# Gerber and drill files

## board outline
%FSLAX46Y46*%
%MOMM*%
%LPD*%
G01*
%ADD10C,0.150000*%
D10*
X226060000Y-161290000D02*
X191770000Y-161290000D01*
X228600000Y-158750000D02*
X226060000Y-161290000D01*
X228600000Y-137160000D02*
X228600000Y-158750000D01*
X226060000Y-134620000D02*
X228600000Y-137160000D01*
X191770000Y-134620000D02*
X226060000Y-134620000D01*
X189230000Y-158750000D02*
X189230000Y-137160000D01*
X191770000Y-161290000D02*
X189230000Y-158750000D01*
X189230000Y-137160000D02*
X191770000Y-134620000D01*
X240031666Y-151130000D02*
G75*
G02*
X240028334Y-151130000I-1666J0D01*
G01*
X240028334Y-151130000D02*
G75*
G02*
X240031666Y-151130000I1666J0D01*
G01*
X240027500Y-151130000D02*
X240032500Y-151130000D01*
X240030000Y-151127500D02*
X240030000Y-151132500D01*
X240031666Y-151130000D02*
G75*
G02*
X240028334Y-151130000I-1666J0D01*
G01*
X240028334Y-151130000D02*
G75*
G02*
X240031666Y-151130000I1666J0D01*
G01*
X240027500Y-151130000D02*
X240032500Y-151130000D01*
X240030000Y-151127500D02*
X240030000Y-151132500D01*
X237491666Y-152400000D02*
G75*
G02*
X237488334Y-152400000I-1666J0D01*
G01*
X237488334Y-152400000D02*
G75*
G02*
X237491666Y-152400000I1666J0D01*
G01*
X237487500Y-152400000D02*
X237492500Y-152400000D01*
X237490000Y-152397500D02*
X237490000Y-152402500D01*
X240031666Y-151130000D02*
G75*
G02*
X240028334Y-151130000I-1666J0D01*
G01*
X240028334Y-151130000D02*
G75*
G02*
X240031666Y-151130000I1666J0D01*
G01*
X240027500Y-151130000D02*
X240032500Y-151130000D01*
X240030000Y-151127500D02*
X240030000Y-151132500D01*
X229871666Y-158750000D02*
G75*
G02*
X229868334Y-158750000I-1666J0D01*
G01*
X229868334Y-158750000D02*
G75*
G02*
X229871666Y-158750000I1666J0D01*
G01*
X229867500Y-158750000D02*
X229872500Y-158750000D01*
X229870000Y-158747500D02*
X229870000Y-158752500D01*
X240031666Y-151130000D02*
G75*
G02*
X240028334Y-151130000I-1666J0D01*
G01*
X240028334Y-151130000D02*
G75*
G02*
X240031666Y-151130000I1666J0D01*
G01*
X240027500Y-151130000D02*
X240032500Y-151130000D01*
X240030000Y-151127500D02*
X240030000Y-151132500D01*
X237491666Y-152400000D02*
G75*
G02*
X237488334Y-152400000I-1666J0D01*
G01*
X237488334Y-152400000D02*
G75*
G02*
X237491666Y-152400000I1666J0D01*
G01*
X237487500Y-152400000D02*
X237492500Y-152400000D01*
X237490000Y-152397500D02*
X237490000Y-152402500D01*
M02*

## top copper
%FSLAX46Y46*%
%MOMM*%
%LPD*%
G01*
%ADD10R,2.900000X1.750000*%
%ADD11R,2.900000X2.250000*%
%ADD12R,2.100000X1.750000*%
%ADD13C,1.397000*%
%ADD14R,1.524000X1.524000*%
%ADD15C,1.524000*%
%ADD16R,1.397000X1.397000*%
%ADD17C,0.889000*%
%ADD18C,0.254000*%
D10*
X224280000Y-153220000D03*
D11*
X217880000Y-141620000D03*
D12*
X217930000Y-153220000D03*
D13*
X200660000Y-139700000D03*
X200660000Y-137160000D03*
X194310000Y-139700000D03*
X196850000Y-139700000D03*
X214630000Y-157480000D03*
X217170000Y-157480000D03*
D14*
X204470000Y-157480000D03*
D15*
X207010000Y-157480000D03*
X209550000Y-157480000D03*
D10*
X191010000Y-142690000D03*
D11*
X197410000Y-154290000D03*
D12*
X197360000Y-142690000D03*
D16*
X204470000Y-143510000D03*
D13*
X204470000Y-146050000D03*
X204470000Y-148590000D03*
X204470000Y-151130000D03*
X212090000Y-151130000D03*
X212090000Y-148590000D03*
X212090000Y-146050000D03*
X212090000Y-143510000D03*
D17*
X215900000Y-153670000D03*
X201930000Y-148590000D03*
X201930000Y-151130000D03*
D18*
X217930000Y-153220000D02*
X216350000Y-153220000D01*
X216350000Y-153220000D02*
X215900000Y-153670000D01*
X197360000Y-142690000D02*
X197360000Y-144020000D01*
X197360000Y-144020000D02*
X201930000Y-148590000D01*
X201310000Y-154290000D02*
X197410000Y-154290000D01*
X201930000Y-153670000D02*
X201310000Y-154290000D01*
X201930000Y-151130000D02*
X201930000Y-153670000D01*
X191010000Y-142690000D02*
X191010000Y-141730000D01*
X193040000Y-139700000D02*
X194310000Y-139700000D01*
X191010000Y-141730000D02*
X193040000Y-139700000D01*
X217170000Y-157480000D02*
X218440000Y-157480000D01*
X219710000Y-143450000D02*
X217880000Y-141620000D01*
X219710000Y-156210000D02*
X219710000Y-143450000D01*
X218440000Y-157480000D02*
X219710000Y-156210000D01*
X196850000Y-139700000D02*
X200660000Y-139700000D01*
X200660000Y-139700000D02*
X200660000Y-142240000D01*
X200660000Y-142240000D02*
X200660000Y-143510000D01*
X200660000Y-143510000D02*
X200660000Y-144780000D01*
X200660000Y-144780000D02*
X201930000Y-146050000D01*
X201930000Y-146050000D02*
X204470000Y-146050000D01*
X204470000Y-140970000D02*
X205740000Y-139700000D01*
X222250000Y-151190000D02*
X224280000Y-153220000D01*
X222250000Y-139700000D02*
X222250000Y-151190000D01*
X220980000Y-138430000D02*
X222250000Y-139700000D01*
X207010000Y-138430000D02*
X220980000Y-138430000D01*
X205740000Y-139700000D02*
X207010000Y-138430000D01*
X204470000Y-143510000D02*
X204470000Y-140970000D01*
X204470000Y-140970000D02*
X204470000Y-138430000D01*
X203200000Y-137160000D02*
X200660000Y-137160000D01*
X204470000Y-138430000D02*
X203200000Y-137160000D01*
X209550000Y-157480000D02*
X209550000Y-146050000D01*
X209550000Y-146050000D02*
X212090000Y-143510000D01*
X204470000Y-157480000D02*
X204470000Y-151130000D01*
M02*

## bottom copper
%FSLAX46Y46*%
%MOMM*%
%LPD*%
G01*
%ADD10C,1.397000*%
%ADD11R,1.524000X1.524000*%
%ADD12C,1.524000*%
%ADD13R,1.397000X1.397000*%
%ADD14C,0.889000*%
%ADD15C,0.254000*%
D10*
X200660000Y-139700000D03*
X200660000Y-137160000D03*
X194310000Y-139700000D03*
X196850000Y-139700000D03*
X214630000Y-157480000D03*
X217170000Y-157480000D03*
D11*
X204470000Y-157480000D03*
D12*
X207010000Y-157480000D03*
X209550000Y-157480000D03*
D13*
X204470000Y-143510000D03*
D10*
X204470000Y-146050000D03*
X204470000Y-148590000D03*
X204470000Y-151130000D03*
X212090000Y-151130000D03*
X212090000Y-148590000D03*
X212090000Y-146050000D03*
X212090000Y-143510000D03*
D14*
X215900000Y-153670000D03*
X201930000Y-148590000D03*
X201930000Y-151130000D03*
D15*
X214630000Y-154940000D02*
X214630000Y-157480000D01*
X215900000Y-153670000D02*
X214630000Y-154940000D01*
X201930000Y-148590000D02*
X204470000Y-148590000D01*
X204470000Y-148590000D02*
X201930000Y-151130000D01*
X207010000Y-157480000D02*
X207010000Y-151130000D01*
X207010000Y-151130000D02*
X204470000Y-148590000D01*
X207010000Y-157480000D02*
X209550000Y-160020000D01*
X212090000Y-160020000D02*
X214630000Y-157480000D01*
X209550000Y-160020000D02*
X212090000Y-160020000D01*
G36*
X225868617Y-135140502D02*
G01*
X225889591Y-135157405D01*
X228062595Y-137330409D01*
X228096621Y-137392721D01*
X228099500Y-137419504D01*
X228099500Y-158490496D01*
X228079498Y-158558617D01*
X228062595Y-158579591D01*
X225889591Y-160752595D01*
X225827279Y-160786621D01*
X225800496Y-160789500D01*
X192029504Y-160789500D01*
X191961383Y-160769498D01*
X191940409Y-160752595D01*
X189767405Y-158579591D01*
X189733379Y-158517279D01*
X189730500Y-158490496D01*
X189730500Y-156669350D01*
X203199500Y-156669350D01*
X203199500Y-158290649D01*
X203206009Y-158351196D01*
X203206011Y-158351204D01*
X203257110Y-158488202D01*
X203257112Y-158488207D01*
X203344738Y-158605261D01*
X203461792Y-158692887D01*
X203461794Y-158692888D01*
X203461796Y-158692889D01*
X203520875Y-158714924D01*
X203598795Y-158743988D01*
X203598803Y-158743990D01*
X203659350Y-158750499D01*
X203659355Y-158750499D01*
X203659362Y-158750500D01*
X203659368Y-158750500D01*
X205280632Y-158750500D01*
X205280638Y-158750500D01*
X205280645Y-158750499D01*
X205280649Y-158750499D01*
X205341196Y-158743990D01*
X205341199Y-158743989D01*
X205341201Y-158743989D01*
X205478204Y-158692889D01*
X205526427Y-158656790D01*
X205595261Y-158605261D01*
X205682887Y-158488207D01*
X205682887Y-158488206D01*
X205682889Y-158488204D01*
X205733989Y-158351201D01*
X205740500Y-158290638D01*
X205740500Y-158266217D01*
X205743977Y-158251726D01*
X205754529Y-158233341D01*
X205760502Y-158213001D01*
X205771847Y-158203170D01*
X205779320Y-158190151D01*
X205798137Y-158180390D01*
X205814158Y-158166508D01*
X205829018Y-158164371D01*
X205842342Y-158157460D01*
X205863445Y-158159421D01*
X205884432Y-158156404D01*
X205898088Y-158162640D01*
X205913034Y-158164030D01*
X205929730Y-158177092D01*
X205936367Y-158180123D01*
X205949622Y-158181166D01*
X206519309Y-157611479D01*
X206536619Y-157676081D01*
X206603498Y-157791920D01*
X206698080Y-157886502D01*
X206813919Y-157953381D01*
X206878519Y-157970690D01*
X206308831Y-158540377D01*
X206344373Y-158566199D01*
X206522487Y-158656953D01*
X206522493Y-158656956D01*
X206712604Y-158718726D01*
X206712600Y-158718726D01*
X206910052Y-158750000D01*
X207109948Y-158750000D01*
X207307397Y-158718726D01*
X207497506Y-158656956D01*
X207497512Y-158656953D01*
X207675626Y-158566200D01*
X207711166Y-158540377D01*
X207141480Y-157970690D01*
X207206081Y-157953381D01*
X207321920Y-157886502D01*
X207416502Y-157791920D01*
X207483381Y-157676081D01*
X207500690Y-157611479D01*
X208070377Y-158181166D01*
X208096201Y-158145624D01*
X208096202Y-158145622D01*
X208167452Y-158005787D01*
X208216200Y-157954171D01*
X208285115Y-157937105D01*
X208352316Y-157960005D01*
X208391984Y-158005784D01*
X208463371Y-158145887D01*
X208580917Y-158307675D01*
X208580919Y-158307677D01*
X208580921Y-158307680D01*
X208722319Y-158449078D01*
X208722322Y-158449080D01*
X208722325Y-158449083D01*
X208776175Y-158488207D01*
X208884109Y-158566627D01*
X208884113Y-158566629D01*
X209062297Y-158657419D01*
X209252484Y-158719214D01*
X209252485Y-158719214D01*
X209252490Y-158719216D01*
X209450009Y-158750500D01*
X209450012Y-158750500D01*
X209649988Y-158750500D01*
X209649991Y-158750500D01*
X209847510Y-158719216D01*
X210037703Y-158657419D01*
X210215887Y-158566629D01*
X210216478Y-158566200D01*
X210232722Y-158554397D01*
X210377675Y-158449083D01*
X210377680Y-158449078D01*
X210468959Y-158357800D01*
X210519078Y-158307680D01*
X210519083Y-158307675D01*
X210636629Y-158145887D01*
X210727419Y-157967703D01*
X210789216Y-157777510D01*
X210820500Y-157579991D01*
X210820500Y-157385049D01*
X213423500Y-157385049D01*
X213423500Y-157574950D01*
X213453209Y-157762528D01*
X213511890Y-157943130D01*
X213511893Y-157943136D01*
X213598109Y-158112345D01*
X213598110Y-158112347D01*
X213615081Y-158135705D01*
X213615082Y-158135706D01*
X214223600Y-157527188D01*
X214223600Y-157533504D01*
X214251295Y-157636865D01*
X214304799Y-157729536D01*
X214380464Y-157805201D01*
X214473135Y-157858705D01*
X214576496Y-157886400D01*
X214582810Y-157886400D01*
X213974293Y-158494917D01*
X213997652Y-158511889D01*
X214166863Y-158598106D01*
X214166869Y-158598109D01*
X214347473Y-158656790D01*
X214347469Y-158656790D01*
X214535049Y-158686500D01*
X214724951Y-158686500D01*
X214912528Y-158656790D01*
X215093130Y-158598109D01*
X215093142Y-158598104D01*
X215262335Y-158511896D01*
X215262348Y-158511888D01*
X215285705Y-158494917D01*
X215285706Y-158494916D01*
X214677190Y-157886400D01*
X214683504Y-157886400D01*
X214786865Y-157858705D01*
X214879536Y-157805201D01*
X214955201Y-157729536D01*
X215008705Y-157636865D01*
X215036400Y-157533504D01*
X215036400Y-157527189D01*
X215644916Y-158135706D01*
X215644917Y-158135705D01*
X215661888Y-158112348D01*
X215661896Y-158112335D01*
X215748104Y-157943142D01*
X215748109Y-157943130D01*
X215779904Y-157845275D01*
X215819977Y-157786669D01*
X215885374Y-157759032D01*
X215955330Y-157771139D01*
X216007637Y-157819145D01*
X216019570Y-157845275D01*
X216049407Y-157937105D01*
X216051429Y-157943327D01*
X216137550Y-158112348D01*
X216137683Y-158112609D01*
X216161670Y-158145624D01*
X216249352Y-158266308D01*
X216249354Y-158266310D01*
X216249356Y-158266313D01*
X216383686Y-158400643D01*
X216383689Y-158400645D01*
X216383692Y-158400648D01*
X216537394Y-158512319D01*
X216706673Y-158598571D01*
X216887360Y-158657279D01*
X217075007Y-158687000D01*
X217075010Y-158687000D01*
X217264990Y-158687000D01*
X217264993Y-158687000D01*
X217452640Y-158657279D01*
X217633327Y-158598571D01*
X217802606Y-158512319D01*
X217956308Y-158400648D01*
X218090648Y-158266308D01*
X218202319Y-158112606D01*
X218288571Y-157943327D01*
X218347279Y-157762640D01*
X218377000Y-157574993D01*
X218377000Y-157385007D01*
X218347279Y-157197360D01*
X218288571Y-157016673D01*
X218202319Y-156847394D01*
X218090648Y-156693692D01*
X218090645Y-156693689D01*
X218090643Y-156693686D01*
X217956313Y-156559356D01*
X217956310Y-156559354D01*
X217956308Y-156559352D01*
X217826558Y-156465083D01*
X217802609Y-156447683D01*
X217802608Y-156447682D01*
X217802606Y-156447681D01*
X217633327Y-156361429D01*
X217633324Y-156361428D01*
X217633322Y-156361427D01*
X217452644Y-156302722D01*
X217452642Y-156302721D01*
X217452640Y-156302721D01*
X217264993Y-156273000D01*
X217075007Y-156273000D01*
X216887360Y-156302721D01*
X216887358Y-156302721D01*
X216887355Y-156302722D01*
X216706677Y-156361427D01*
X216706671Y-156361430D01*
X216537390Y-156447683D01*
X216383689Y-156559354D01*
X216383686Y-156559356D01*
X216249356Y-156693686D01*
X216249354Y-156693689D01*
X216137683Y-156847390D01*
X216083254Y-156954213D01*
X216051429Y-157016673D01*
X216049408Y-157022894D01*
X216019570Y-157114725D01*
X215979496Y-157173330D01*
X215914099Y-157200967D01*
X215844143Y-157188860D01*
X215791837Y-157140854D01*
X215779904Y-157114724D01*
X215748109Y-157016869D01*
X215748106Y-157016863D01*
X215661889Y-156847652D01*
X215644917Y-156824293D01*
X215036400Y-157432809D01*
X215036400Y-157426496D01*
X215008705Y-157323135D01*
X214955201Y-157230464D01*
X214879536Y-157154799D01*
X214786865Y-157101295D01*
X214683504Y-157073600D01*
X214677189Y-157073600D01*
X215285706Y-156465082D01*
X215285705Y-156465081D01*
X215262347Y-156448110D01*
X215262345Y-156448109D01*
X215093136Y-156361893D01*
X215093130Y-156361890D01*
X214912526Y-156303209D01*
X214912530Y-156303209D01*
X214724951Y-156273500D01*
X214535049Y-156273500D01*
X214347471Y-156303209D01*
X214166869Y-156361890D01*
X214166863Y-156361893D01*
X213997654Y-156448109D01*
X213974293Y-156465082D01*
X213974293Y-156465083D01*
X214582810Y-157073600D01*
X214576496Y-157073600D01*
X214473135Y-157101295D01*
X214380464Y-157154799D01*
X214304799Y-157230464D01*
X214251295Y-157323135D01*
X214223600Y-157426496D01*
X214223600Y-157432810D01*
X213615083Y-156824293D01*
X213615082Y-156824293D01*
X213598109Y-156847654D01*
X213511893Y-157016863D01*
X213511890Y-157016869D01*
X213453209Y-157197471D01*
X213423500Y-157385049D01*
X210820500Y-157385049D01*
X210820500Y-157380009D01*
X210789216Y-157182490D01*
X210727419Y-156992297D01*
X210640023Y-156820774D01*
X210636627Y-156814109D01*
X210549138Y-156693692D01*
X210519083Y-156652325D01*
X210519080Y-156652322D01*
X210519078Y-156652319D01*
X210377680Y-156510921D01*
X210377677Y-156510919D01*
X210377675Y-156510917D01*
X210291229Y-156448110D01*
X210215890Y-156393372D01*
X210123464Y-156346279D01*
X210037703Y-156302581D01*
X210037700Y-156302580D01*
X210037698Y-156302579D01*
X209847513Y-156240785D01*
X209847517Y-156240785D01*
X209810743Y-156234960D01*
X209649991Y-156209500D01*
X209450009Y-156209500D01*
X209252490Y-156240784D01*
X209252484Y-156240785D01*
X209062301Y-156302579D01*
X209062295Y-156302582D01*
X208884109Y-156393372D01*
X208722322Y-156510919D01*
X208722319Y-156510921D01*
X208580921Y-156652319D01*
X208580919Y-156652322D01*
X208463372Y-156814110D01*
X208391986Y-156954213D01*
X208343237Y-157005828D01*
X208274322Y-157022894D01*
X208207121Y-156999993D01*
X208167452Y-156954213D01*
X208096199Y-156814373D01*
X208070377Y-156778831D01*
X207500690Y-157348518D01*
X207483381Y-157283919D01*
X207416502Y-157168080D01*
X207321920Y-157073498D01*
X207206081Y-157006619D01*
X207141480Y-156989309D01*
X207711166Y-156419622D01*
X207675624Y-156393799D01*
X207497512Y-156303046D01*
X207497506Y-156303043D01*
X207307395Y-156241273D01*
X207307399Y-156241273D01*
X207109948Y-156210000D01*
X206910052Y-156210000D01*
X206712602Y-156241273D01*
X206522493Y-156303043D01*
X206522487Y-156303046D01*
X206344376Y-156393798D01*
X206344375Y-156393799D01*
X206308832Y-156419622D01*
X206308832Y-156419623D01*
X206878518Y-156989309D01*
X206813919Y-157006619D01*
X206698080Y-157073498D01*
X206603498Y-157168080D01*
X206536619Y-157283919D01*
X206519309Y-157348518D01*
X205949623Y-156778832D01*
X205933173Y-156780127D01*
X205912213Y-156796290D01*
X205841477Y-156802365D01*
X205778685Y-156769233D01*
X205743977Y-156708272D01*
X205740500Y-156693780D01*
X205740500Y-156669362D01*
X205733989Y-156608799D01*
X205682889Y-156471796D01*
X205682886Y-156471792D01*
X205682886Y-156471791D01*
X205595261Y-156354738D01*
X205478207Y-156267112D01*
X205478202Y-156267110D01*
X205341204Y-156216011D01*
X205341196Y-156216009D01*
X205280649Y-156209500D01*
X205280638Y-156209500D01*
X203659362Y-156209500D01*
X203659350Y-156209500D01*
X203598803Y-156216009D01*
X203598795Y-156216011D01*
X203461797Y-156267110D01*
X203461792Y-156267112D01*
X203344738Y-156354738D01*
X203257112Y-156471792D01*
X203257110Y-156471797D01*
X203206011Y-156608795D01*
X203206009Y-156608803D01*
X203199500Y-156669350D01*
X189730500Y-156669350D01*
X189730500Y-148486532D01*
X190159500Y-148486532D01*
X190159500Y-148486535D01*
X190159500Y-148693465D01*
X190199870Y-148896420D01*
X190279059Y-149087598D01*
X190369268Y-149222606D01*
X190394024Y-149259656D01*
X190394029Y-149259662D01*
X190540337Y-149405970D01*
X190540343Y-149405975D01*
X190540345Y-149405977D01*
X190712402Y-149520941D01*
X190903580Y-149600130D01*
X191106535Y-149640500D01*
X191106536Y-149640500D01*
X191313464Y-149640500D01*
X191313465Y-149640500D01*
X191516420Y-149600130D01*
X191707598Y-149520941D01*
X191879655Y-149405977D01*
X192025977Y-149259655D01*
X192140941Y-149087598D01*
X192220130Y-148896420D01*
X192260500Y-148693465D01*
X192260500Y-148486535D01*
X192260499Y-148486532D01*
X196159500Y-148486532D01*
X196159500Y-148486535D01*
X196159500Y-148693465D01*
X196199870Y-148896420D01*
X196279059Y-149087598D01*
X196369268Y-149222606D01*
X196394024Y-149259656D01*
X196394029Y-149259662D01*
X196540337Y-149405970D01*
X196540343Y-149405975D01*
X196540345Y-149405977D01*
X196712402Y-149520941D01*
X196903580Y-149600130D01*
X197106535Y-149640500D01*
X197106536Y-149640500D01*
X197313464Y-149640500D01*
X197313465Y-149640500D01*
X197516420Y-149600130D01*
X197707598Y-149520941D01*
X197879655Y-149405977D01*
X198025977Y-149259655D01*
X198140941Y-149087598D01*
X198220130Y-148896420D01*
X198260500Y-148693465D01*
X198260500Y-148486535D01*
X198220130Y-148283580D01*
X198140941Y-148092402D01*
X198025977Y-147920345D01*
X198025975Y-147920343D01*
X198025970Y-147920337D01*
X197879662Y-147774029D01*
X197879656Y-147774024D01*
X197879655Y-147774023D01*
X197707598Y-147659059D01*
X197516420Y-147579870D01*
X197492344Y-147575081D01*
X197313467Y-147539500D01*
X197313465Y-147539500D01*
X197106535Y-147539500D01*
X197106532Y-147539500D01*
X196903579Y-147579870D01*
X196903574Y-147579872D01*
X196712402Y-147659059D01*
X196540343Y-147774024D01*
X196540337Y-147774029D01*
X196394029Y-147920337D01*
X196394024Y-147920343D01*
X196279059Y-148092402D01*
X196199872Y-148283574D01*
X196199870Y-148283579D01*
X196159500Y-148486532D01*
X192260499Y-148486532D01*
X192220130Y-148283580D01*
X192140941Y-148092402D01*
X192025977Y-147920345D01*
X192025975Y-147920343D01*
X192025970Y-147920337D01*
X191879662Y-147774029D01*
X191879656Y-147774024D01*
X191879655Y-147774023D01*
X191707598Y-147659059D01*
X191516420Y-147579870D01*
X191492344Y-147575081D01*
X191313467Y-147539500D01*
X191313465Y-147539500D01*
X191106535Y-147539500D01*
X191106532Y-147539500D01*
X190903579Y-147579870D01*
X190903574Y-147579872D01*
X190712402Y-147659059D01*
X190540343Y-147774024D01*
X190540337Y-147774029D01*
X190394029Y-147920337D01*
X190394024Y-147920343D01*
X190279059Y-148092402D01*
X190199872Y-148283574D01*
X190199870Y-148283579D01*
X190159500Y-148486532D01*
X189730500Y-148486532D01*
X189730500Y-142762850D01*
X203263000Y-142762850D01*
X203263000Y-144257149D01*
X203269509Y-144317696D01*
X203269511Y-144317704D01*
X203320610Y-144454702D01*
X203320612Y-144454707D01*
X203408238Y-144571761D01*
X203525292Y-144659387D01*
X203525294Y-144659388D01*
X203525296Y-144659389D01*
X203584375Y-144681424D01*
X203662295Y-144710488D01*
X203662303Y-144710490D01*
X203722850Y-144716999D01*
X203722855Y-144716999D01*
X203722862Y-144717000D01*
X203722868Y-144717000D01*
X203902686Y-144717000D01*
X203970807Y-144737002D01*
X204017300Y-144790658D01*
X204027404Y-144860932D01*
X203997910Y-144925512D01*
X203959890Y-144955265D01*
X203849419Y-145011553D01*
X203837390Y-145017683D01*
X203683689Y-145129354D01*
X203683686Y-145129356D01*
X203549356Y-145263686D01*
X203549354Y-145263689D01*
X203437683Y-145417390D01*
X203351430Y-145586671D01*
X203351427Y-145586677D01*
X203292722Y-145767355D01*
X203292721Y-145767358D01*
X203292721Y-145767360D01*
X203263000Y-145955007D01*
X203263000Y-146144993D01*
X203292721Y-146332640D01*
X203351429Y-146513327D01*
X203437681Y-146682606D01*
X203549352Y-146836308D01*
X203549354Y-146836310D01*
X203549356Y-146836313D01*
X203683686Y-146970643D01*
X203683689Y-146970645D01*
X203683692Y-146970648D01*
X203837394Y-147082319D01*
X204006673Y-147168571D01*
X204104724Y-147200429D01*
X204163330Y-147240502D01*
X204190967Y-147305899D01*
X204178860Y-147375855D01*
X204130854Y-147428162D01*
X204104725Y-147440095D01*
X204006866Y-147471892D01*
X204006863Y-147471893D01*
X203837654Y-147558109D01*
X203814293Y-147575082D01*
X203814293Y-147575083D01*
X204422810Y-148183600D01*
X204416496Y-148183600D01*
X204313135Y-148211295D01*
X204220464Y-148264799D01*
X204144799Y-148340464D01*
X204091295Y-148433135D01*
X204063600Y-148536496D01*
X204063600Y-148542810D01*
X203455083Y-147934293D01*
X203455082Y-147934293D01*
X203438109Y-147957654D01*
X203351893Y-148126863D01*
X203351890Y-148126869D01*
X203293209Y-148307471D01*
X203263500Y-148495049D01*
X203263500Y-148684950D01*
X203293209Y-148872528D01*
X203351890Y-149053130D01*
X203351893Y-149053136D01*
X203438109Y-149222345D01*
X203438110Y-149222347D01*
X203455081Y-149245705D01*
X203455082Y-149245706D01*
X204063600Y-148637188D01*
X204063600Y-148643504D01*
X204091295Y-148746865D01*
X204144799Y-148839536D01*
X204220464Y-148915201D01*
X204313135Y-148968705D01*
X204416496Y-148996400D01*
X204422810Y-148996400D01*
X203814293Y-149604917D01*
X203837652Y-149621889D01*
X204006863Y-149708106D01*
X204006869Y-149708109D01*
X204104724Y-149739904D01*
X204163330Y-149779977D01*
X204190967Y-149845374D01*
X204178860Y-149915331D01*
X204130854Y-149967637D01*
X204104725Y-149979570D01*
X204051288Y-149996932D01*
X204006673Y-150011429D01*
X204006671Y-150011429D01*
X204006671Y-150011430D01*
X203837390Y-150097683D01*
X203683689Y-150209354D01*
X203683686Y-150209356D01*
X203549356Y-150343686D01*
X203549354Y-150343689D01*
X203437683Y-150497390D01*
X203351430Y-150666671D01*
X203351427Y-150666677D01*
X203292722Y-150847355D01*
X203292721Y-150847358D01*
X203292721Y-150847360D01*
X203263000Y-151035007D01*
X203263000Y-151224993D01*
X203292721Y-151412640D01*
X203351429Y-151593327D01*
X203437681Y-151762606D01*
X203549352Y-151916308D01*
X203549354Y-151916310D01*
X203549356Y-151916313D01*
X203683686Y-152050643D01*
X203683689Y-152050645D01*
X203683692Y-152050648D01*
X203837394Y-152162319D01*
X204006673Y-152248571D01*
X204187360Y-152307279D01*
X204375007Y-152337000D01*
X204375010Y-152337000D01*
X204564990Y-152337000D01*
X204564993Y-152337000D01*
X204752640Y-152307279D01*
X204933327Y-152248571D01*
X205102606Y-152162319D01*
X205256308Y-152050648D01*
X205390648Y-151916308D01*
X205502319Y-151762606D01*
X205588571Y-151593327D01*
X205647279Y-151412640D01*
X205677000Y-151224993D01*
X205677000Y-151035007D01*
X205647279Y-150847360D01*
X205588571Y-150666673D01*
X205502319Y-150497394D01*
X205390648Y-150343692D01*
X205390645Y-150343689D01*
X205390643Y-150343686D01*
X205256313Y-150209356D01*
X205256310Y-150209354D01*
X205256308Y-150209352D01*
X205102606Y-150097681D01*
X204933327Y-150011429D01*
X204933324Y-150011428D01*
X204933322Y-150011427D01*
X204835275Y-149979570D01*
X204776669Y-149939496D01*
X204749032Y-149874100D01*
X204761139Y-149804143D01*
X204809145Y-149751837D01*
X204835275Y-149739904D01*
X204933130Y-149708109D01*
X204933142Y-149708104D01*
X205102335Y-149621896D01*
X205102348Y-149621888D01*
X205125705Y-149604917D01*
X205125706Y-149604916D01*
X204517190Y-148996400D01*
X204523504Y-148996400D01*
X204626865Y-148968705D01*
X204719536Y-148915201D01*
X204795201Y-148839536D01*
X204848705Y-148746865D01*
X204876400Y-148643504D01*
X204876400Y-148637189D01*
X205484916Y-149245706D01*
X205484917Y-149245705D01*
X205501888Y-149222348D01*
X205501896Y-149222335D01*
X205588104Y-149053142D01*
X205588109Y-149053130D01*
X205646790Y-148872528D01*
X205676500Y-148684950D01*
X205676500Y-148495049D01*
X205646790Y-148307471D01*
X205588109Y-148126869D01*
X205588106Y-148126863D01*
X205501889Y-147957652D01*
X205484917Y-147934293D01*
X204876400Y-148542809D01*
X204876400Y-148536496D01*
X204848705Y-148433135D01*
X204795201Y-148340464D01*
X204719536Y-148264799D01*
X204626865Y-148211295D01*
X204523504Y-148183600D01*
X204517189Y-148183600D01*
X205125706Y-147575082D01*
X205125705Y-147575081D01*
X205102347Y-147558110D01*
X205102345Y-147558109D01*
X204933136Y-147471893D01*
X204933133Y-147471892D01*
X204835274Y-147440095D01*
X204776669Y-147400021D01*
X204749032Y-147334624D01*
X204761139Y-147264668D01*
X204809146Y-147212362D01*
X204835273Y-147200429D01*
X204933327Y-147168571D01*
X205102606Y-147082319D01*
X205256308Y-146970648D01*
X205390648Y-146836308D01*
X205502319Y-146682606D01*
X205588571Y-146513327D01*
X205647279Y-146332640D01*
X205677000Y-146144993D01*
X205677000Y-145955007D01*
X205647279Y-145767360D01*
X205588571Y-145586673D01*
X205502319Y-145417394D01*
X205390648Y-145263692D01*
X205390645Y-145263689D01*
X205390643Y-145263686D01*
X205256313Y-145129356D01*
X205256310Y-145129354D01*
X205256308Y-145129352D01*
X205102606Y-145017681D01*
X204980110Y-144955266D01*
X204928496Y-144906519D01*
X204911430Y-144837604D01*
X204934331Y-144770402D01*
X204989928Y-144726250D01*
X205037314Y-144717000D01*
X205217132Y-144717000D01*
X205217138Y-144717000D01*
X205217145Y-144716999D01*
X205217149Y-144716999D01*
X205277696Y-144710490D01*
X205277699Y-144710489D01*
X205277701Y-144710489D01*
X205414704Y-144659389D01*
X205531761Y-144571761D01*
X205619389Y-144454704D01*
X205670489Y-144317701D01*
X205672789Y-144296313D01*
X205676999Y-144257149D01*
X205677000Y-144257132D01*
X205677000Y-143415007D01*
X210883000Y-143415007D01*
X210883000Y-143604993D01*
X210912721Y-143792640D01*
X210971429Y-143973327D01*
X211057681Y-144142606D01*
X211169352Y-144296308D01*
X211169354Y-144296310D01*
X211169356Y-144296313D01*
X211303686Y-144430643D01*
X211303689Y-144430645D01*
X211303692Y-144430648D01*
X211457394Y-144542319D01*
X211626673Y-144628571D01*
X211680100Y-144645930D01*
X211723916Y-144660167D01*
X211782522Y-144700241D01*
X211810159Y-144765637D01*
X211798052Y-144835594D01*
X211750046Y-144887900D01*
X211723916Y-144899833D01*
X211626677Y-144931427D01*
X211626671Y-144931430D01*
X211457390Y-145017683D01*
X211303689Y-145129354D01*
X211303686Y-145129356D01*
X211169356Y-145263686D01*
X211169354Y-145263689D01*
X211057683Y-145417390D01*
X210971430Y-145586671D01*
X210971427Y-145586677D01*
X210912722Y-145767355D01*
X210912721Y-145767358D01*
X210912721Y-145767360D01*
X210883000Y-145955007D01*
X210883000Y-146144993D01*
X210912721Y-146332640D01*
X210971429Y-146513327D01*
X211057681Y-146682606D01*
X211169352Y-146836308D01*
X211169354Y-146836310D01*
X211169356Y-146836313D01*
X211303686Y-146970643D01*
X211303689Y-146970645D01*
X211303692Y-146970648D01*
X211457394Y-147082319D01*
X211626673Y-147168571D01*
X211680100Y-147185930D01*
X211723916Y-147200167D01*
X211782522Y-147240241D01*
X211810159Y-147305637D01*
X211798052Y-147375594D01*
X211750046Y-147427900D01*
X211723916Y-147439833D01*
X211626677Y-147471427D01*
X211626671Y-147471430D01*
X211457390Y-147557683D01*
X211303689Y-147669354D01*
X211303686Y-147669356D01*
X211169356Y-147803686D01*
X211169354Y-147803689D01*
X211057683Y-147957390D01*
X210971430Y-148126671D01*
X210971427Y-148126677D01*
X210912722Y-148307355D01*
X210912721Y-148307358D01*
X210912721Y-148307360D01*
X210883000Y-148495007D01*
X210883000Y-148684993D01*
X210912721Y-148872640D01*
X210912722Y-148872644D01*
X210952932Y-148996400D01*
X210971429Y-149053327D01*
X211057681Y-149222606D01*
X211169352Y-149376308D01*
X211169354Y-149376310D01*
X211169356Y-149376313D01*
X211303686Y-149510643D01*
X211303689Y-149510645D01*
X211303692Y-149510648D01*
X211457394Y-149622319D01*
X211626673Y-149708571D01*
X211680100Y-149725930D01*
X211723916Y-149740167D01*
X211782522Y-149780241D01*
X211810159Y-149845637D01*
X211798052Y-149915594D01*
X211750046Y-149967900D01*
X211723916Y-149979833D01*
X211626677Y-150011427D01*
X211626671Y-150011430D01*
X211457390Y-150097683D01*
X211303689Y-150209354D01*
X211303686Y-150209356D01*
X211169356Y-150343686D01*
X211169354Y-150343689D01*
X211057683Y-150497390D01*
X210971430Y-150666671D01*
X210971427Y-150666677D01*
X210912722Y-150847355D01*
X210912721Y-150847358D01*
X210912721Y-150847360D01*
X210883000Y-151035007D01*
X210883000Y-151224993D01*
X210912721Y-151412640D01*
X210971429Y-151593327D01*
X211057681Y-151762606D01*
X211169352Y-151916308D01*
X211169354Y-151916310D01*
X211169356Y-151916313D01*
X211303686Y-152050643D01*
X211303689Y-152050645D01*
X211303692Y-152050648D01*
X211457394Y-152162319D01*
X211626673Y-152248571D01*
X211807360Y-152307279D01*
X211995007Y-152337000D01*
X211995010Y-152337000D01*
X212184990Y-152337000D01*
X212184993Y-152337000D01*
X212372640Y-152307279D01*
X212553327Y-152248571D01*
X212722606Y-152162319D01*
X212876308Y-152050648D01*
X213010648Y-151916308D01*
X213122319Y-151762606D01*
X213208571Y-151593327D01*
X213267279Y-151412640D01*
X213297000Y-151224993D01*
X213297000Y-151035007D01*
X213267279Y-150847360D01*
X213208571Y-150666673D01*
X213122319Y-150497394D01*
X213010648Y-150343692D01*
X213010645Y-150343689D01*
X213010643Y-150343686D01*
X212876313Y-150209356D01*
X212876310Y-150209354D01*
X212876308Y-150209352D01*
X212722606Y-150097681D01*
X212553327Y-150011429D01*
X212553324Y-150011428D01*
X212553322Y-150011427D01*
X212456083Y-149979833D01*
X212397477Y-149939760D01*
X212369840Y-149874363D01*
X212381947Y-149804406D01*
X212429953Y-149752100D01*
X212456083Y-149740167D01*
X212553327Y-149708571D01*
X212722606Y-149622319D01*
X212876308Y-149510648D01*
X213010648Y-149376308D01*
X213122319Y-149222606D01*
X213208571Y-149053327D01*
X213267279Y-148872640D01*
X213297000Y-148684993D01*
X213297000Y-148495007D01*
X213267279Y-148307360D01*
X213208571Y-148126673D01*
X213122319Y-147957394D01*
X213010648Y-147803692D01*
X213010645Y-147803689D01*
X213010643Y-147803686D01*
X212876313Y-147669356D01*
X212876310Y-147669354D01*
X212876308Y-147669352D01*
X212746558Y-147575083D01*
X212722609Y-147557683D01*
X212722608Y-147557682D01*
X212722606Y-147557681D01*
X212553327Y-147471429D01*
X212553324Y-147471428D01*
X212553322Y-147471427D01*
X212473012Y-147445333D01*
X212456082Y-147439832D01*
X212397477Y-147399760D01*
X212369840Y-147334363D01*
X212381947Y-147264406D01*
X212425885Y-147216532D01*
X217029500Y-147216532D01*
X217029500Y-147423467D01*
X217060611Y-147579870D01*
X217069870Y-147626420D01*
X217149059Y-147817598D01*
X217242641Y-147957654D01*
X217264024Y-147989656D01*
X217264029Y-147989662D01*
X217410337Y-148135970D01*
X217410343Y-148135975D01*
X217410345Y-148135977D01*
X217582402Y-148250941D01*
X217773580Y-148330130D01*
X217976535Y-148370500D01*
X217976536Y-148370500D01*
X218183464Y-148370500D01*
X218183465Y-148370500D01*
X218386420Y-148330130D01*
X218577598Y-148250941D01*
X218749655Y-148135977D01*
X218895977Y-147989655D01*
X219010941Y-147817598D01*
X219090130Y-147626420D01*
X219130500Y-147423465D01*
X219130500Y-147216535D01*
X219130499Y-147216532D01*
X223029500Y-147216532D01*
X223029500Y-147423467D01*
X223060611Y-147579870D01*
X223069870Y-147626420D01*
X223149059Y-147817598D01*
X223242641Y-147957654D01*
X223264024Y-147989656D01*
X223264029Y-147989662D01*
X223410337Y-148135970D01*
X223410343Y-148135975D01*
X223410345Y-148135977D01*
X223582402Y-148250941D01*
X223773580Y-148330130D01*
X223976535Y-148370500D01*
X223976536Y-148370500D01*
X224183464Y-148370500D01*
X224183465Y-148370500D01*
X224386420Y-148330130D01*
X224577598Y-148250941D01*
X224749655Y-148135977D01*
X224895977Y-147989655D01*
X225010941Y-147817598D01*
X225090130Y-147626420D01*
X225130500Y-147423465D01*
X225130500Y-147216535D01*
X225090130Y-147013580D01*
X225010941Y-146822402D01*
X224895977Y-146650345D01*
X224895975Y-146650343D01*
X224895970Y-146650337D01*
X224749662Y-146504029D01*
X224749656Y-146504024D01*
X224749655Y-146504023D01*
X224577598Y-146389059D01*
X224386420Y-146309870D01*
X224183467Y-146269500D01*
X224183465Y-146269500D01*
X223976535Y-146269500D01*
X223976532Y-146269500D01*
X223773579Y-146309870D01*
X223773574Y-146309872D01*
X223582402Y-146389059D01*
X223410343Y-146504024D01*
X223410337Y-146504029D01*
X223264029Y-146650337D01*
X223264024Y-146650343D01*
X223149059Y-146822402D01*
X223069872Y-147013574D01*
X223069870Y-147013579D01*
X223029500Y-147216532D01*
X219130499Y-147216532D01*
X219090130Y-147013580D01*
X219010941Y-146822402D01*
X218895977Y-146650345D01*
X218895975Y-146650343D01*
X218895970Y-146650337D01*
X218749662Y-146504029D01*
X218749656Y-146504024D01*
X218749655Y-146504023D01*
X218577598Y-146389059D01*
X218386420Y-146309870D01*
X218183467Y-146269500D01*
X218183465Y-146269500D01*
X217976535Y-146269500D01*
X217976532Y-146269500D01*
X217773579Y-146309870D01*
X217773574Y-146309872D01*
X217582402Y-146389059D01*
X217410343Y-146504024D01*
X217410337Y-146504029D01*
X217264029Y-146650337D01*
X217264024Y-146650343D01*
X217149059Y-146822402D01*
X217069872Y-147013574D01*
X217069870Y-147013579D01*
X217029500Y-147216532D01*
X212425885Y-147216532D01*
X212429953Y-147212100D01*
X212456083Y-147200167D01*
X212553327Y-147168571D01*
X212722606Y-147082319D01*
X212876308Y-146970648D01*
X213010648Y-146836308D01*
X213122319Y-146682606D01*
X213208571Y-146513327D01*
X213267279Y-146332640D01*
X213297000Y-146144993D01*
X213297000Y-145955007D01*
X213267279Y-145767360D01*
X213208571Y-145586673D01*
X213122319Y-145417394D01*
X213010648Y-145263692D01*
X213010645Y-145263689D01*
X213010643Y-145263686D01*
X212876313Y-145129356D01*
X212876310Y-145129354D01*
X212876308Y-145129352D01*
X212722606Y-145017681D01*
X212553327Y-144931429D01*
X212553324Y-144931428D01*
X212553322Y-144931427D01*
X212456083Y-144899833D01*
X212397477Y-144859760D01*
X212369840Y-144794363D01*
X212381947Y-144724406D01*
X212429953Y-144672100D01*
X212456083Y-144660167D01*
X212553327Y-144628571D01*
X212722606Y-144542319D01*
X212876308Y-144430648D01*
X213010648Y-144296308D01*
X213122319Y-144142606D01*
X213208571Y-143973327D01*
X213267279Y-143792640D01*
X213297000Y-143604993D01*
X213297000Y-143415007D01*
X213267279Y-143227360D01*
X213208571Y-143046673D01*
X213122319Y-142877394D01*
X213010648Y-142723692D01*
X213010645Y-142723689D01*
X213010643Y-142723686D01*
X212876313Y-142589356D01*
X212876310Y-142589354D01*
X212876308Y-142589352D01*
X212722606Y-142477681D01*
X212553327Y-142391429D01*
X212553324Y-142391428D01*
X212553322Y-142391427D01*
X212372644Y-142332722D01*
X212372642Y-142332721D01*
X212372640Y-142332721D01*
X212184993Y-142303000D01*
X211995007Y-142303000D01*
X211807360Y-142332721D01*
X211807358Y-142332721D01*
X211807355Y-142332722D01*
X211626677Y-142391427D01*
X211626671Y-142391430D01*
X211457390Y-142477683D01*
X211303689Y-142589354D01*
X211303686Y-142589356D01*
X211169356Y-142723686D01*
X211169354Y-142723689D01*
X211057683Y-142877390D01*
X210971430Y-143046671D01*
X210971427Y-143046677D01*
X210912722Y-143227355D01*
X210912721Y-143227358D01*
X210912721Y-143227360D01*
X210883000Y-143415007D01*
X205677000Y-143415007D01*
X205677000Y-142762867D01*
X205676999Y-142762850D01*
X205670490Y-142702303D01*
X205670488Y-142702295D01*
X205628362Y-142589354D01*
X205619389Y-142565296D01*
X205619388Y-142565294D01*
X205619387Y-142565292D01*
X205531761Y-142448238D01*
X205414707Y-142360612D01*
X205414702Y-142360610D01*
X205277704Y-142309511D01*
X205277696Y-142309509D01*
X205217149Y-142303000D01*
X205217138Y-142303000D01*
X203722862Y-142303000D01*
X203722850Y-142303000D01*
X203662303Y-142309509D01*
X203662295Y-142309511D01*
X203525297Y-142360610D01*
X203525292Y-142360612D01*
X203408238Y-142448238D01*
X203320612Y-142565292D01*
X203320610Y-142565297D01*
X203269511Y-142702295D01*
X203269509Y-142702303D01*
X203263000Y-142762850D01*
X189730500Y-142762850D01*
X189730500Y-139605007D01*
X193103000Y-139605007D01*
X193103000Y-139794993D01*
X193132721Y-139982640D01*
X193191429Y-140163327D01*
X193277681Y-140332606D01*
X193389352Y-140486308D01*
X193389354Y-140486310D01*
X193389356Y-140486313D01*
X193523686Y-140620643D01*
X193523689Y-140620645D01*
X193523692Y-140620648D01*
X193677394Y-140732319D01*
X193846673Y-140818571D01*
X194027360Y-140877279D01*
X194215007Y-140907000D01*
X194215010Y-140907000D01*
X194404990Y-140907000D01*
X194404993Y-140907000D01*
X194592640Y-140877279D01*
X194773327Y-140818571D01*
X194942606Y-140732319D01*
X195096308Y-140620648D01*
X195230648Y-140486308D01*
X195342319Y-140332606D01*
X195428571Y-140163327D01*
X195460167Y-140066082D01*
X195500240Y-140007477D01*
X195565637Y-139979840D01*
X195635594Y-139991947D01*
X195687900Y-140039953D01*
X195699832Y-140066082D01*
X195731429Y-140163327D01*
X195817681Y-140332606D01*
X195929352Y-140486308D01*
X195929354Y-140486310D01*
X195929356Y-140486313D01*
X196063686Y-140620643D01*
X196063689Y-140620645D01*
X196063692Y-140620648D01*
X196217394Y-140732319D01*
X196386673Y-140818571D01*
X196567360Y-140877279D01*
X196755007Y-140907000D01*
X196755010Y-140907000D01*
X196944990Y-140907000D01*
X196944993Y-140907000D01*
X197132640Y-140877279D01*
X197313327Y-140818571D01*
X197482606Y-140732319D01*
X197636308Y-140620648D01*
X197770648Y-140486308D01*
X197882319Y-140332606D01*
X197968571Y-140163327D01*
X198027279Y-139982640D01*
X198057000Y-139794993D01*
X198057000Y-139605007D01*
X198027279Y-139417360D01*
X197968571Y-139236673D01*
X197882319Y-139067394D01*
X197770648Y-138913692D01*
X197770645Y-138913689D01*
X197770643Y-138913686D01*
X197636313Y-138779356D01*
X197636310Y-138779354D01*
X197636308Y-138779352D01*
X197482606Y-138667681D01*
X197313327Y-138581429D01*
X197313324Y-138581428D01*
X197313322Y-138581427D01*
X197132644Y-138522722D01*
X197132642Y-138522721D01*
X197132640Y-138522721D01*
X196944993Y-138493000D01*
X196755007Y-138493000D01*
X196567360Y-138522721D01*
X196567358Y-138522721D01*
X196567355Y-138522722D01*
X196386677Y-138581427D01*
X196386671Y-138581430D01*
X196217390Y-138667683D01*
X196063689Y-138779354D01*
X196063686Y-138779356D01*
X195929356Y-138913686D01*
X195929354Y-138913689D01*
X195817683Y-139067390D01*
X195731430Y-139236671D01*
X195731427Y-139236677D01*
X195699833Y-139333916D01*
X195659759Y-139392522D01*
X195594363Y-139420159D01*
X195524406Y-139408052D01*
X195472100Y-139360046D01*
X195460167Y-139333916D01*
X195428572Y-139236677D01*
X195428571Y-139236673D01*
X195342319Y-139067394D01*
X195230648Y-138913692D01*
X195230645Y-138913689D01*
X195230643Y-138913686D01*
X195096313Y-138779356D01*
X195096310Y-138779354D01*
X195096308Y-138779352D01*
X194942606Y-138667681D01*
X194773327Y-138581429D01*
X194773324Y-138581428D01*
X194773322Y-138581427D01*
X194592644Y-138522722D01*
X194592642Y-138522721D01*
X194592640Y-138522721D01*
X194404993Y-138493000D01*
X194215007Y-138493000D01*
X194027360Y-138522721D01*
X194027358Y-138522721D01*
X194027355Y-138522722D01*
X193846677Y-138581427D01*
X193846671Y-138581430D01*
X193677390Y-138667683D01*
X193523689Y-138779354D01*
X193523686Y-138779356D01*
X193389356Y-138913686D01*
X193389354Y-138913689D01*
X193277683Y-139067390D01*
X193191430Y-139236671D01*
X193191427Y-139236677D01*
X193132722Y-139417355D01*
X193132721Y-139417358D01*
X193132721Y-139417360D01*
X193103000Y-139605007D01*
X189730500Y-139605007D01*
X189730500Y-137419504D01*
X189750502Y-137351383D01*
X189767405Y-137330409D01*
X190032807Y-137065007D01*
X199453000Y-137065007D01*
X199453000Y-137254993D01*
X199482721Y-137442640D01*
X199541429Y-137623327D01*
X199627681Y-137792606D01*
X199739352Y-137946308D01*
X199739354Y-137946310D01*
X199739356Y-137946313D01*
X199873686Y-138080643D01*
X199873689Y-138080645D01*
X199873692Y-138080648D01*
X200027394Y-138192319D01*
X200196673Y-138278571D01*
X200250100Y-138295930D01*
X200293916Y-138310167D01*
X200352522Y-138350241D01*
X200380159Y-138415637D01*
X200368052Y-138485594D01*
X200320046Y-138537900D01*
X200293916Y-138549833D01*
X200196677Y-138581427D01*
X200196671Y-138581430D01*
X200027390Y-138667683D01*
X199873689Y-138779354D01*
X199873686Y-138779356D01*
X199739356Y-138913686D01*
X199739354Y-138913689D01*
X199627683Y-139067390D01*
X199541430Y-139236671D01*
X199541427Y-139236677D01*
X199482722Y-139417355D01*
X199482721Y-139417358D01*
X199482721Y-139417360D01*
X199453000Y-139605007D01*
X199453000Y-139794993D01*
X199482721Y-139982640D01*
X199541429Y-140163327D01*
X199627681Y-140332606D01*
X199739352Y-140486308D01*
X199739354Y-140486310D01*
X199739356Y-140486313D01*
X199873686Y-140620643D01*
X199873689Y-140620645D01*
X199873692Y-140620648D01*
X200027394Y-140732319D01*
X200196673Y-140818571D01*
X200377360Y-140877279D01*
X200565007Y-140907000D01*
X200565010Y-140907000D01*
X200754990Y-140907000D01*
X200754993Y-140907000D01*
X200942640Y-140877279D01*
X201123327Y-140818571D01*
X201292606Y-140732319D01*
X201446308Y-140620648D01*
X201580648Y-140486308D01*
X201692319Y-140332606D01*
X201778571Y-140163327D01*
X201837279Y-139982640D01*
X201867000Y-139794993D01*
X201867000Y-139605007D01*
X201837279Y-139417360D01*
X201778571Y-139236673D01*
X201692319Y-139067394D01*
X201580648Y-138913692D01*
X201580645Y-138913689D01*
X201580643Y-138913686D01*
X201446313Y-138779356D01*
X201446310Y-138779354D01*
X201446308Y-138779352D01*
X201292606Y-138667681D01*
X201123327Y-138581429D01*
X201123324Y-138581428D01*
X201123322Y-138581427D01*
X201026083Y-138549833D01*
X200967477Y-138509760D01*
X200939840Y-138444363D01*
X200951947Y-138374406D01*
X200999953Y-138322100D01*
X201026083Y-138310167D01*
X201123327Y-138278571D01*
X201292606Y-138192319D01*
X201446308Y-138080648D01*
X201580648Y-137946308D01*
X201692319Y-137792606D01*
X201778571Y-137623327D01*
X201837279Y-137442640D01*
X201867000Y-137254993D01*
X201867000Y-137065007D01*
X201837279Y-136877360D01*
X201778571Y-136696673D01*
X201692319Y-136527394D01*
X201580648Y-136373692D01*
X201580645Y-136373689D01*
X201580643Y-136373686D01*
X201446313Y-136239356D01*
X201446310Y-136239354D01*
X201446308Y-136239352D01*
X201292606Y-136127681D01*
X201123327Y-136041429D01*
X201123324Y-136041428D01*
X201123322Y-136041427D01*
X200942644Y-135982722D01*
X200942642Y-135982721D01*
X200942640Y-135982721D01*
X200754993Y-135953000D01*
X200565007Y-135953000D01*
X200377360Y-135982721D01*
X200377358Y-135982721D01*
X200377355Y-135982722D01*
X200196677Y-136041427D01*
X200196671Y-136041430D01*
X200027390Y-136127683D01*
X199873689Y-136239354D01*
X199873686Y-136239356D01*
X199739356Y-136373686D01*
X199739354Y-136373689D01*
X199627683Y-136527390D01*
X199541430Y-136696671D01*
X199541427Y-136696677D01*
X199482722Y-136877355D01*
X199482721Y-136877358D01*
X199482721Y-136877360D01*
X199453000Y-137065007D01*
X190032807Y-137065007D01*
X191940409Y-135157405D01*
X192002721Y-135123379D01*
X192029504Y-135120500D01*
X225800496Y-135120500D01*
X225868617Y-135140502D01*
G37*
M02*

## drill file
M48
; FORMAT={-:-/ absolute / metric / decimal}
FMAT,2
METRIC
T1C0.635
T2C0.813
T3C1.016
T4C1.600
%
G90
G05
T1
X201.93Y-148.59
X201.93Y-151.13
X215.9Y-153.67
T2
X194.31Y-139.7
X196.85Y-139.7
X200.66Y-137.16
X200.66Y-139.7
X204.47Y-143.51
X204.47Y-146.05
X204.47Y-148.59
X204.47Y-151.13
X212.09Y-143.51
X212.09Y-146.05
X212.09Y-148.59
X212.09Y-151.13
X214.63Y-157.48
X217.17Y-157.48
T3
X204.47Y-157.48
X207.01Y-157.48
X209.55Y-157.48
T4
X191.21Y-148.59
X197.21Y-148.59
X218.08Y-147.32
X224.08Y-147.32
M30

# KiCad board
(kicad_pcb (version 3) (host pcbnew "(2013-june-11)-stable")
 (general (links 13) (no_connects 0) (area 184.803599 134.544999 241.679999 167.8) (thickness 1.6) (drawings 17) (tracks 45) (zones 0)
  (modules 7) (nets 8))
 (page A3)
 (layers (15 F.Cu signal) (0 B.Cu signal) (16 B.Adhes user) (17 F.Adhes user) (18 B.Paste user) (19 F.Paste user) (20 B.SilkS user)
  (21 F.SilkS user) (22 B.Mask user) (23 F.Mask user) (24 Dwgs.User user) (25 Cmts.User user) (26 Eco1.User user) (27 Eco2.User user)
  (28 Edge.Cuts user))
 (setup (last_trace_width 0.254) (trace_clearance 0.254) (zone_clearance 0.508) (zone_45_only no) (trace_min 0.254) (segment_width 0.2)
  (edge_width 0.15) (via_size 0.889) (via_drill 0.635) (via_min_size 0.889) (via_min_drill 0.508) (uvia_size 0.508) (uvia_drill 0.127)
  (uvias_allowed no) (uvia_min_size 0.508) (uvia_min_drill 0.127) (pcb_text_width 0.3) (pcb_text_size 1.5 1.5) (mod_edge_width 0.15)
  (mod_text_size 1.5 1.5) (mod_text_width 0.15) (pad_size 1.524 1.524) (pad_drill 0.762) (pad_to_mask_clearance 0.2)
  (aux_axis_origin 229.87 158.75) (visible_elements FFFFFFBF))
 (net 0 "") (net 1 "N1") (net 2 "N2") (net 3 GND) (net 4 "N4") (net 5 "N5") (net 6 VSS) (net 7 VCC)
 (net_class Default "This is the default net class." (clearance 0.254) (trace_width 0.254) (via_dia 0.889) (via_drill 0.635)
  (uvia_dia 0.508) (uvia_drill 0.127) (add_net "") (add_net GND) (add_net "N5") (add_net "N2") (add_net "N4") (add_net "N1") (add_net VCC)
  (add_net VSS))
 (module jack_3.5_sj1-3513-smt (layer F.Cu) (at 220.98 147.32 90)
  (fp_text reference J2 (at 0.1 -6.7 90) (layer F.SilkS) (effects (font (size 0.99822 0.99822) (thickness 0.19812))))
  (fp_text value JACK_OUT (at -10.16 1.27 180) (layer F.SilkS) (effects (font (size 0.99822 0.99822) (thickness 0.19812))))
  (pad "" np_thru_hole circle (at 0 3.1 90) (size 1.6 1.6) (drill 1.6) (layers *.Cu *.Mask F.SilkS))
  (pad "" np_thru_hole circle (at 0 -2.9 90) (size 1.6 1.6) (drill 1.6) (layers *.Cu *.Mask F.SilkS))
  (pad 1 smd rect (at -5.9 3.3 90) (size 1.75 2.9) (layers F.Cu F.Paste F.Mask) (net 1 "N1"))
  (pad 2 smd rect (at 5.7 -3.1 90) (size 2.25 2.9) (layers F.Cu F.Paste F.Mask) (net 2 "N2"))
  (pad 3 smd rect (at -5.9 -3.05 90) (size 1.75 2.1) (layers F.Cu F.Paste F.Mask) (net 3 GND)))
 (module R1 (layer F.Cu) (at 200.66 138.43 90) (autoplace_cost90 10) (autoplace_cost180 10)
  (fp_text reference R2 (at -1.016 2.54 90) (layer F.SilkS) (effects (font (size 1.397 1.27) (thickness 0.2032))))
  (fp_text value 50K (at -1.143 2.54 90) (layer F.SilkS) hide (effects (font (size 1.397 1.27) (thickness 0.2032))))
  (pad 1 thru_hole circle (at -1.27 0 90) (size 1.397 1.397) (drill 0.8128) (layers *.Cu *.Mask F.SilkS) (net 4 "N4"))
  (pad 2 thru_hole circle (at 1.27 0 90) (size 1.397 1.397) (drill 0.8128) (layers *.Cu *.Mask F.SilkS) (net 1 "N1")))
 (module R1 (layer F.Cu) (at 195.58 139.7) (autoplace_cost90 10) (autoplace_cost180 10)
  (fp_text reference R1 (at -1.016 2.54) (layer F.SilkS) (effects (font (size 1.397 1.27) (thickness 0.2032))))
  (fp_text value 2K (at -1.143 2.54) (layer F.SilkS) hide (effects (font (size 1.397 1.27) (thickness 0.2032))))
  (pad 1 thru_hole circle (at -1.27 0) (size 1.397 1.397) (drill 0.8128) (layers *.Cu *.Mask F.SilkS) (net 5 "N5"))
  (pad 2 thru_hole circle (at 1.27 0) (size 1.397 1.397) (drill 0.8128) (layers *.Cu *.Mask F.SilkS) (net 4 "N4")))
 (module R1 (layer F.Cu) (at 215.9 157.48) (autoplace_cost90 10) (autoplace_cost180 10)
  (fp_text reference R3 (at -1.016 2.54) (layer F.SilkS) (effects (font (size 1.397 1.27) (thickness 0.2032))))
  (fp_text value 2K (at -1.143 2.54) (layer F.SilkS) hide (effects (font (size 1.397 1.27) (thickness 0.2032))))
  (pad 1 thru_hole circle (at -1.27 0) (size 1.397 1.397) (drill 0.8128) (layers *.Cu *.Mask F.SilkS) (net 3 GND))
  (pad 2 thru_hole circle (at 1.27 0) (size 1.397 1.397) (drill 0.8128) (layers *.Cu *.Mask F.SilkS) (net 2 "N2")))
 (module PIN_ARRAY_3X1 (layer F.Cu) (at 207.01 157.48)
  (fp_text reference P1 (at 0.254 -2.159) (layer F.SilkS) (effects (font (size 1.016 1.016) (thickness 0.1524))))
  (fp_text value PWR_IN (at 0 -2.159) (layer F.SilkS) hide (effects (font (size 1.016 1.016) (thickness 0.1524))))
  (pad 1 thru_hole rect (at -2.54 0) (size 1.524 1.524) (drill 1.016) (layers *.Cu *.Mask F.SilkS) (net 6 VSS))
  (pad 2 thru_hole circle (at 0 0) (size 1.524 1.524) (drill 1.016) (layers *.Cu *.Mask F.SilkS) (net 3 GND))
  (pad 3 thru_hole circle (at 2.54 0) (size 1.524 1.524) (drill 1.016) (layers *.Cu *.Mask F.SilkS) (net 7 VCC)))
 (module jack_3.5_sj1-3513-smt (layer F.Cu) (at 194.31 148.59 270)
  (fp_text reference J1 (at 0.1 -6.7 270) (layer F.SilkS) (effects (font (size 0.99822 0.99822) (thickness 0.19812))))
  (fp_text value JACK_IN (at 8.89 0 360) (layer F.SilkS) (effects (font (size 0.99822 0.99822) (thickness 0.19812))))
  (pad "" np_thru_hole circle (at 0 3.1 270) (size 1.6 1.6) (drill 1.6) (layers *.Cu *.Mask F.SilkS))
  (pad "" np_thru_hole circle (at 0 -2.9 270) (size 1.6 1.6) (drill 1.6) (layers *.Cu *.Mask F.SilkS))
  (pad 1 smd rect (at -5.9 3.3 270) (size 1.75 2.9) (layers F.Cu F.Paste F.Mask) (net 5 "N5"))
  (pad 2 smd rect (at 5.7 -3.1 270) (size 2.25 2.9) (layers F.Cu F.Paste F.Mask) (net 3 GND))
  (pad 3 smd rect (at -5.9 -3.05 270) (size 1.75 2.1) (layers F.Cu F.Paste F.Mask) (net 3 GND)))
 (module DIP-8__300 (layer F.Cu) (at 208.28 147.32 270)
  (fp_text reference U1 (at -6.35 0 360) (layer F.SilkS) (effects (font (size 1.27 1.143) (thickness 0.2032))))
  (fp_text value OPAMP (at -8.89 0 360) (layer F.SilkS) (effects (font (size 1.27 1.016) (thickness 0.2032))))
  (pad 1 thru_hole rect (at -3.81 3.81 270) (size 1.397 1.397) (drill 0.8128) (layers *.Cu *.Mask F.SilkS) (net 1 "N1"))
  (pad 2 thru_hole circle (at -1.27 3.81 270) (size 1.397 1.397) (drill 0.8128) (layers *.Cu *.Mask F.SilkS) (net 4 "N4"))
  (pad 3 thru_hole circle (at 1.27 3.81 270) (size 1.397 1.397) (drill 0.8128) (layers *.Cu *.Mask F.SilkS) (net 3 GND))
  (pad 4 thru_hole circle (at 3.81 3.81 270) (size 1.397 1.397) (drill 0.8128) (layers *.Cu *.Mask F.SilkS) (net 6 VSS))
  (pad 5 thru_hole circle (at 3.81 -3.81 270) (size 1.397 1.397) (drill 0.8128) (layers *.Cu *.Mask F.SilkS))
  (pad 6 thru_hole circle (at 1.27 -3.81 270) (size 1.397 1.397) (drill 0.8128) (layers *.Cu *.Mask F.SilkS))
  (pad 7 thru_hole circle (at -1.27 -3.81 270) (size 1.397 1.397) (drill 0.8128) (layers *.Cu *.Mask F.SilkS))
  (pad 8 thru_hole circle (at -3.81 -3.81 270) (size 1.397 1.397) (drill 0.8128) (layers *.Cu *.Mask F.SilkS) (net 7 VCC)))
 (gr_line (start 226.06 161.29) (end 191.77 161.29) (angle 90) (layer Edge.Cuts) (width 0.15))
 (gr_line (start 228.6 158.75) (end 226.06 161.29) (angle 90) (layer Edge.Cuts) (width 0.15))
 (gr_line (start 228.6 137.16) (end 228.6 158.75) (angle 90) (layer Edge.Cuts) (width 0.15))
 (gr_line (start 226.06 134.62) (end 228.6 137.16) (angle 90) (layer Edge.Cuts) (width 0.15))
 (gr_line (start 191.77 134.62) (end 226.06 134.62) (angle 90) (layer Edge.Cuts) (width 0.15))
 (gr_line (start 189.23 158.75) (end 189.23 137.16) (angle 90) (layer Edge.Cuts) (width 0.15))
 (gr_line (start 191.77 161.29) (end 189.23 158.75) (angle 90) (layer Edge.Cuts) (width 0.15))
 (gr_line (start 189.23 137.16) (end 191.77 134.62) (angle 90) (layer Edge.Cuts) (width 0.15))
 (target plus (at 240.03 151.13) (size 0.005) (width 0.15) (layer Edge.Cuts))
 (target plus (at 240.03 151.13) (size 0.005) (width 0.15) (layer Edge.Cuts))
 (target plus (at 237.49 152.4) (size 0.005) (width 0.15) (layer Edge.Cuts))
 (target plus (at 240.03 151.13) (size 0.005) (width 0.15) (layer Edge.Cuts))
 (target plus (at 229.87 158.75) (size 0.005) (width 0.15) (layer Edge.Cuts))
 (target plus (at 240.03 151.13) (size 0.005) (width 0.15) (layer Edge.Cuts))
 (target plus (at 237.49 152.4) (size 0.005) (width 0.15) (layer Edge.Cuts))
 (segment (start 217.93 153.22) (end 216.35 153.22) (width 0.254) (layer F.Cu) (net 3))
 (segment (start 214.63 154.94) (end 214.63 157.48) (width 0.254) (layer B.Cu) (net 3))
 (segment (start 215.9 153.67) (end 214.63 154.94) (width 0.254) (layer B.Cu) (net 3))
 (via (at 215.9 153.67) (size 0.889) (layers F.Cu B.Cu) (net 3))
 (segment (start 216.35 153.22) (end 215.9 153.67) (width 0.254) (layer F.Cu) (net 3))
 (segment (start 197.36 142.69) (end 197.36 144.02) (width 0.254) (layer F.Cu) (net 3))
 (segment (start 201.93 148.59) (end 204.47 148.59) (width 0.254) (layer B.Cu) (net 3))
 (via (at 201.93 148.59) (size 0.889) (layers F.Cu B.Cu) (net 3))
 (segment (start 197.36 144.02) (end 201.93 148.59) (width 0.254) (layer F.Cu) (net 3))
 (segment (start 204.47 148.59) (end 201.93 151.13) (width 0.254) (layer B.Cu) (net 3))
 (segment (start 201.31 154.29) (end 197.41 154.29) (width 0.254) (layer F.Cu) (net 3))
 (segment (start 201.93 153.67) (end 201.31 154.29) (width 0.254) (layer F.Cu) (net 3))
 (segment (start 201.93 151.13) (end 201.93 153.67) (width 0.254) (layer F.Cu) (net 3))
 (via (at 201.93 151.13) (size 0.889) (layers F.Cu B.Cu) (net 3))
 (segment (start 207.01 157.48) (end 207.01 151.13) (width 0.254) (layer B.Cu) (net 3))
 (segment (start 207.01 151.13) (end 204.47 148.59) (width 0.254) (layer B.Cu) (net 3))
 (segment (start 207.01 157.48) (end 209.55 160.02) (width 0.254) (layer B.Cu) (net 3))
 (segment (start 212.09 160.02) (end 214.63 157.48) (width 0.254) (layer B.Cu) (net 3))
 (segment (start 209.55 160.02) (end 212.09 160.02) (width 0.254) (layer B.Cu) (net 3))
 (segment (start 191.01 142.69) (end 191.01 141.73) (width 0.254) (layer F.Cu) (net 5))
 (segment (start 193.04 139.7) (end 194.31 139.7) (width 0.254) (layer F.Cu) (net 5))
 (segment (start 191.01 141.73) (end 193.04 139.7) (width 0.254) (layer F.Cu) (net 5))
 (segment (start 217.17 157.48) (end 218.44 157.48) (width 0.254) (layer F.Cu) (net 2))
 (segment (start 219.71 143.45) (end 217.88 141.62) (width 0.254) (layer F.Cu) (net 2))
 (segment (start 219.71 156.21) (end 219.71 143.45) (width 0.254) (layer F.Cu) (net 2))
 (segment (start 218.44 157.48) (end 219.71 156.21) (width 0.254) (layer F.Cu) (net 2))
 (segment (start 196.85 139.7) (end 200.66 139.7) (width 0.254) (layer F.Cu) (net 4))
 (segment (start 200.66 139.7) (end 200.66 142.24) (width 0.254) (layer F.Cu) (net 4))
 (segment (start 200.66 142.24) (end 200.66 143.51) (width 0.254) (layer F.Cu) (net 4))
 (segment (start 200.66 143.51) (end 200.66 144.78) (width 0.254) (layer F.Cu) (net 4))
 (segment (start 200.66 144.78) (end 201.93 146.05) (width 0.254) (layer F.Cu) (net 4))
 (segment (start 201.93 146.05) (end 204.47 146.05) (width 0.254) (layer F.Cu) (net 4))
 (segment (start 204.47 140.97) (end 205.74 139.7) (width 0.254) (layer F.Cu) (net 1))
 (segment (start 222.25 151.19) (end 224.28 153.22) (width 0.254) (layer F.Cu) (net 1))
 (segment (start 222.25 139.7) (end 222.25 151.19) (width 0.254) (layer F.Cu) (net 1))
 (segment (start 220.98 138.43) (end 222.25 139.7) (width 0.254) (layer F.Cu) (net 1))
 (segment (start 207.01 138.43) (end 220.98 138.43) (width 0.254) (layer F.Cu) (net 1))
 (segment (start 205.74 139.7) (end 207.01 138.43) (width 0.254) (layer F.Cu) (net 1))
 (segment (start 204.47 143.51) (end 204.47 140.97) (width 0.254) (layer F.Cu) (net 1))
 (segment (start 204.47 140.97) (end 204.47 138.43) (width 0.254) (layer F.Cu) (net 1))
 (segment (start 203.2 137.16) (end 200.66 137.16) (width 0.254) (layer F.Cu) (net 1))
 (segment (start 204.47 138.43) (end 203.2 137.16) (width 0.254) (layer F.Cu) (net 1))
 (segment (start 209.55 157.48) (end 209.55 146.05) (width 0.254) (layer F.Cu) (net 7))
 (segment (start 209.55 146.05) (end 212.09 143.51) (width 0.254) (layer F.Cu) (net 7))
 (segment (start 204.47 157.48) (end 204.47 151.13) (width 0.254) (layer F.Cu) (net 6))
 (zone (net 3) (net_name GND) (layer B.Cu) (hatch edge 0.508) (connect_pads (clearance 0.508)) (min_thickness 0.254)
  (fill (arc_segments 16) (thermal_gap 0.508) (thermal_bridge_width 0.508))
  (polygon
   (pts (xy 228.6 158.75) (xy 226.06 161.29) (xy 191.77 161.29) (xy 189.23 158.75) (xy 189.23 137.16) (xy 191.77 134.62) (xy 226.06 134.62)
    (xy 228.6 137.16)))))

